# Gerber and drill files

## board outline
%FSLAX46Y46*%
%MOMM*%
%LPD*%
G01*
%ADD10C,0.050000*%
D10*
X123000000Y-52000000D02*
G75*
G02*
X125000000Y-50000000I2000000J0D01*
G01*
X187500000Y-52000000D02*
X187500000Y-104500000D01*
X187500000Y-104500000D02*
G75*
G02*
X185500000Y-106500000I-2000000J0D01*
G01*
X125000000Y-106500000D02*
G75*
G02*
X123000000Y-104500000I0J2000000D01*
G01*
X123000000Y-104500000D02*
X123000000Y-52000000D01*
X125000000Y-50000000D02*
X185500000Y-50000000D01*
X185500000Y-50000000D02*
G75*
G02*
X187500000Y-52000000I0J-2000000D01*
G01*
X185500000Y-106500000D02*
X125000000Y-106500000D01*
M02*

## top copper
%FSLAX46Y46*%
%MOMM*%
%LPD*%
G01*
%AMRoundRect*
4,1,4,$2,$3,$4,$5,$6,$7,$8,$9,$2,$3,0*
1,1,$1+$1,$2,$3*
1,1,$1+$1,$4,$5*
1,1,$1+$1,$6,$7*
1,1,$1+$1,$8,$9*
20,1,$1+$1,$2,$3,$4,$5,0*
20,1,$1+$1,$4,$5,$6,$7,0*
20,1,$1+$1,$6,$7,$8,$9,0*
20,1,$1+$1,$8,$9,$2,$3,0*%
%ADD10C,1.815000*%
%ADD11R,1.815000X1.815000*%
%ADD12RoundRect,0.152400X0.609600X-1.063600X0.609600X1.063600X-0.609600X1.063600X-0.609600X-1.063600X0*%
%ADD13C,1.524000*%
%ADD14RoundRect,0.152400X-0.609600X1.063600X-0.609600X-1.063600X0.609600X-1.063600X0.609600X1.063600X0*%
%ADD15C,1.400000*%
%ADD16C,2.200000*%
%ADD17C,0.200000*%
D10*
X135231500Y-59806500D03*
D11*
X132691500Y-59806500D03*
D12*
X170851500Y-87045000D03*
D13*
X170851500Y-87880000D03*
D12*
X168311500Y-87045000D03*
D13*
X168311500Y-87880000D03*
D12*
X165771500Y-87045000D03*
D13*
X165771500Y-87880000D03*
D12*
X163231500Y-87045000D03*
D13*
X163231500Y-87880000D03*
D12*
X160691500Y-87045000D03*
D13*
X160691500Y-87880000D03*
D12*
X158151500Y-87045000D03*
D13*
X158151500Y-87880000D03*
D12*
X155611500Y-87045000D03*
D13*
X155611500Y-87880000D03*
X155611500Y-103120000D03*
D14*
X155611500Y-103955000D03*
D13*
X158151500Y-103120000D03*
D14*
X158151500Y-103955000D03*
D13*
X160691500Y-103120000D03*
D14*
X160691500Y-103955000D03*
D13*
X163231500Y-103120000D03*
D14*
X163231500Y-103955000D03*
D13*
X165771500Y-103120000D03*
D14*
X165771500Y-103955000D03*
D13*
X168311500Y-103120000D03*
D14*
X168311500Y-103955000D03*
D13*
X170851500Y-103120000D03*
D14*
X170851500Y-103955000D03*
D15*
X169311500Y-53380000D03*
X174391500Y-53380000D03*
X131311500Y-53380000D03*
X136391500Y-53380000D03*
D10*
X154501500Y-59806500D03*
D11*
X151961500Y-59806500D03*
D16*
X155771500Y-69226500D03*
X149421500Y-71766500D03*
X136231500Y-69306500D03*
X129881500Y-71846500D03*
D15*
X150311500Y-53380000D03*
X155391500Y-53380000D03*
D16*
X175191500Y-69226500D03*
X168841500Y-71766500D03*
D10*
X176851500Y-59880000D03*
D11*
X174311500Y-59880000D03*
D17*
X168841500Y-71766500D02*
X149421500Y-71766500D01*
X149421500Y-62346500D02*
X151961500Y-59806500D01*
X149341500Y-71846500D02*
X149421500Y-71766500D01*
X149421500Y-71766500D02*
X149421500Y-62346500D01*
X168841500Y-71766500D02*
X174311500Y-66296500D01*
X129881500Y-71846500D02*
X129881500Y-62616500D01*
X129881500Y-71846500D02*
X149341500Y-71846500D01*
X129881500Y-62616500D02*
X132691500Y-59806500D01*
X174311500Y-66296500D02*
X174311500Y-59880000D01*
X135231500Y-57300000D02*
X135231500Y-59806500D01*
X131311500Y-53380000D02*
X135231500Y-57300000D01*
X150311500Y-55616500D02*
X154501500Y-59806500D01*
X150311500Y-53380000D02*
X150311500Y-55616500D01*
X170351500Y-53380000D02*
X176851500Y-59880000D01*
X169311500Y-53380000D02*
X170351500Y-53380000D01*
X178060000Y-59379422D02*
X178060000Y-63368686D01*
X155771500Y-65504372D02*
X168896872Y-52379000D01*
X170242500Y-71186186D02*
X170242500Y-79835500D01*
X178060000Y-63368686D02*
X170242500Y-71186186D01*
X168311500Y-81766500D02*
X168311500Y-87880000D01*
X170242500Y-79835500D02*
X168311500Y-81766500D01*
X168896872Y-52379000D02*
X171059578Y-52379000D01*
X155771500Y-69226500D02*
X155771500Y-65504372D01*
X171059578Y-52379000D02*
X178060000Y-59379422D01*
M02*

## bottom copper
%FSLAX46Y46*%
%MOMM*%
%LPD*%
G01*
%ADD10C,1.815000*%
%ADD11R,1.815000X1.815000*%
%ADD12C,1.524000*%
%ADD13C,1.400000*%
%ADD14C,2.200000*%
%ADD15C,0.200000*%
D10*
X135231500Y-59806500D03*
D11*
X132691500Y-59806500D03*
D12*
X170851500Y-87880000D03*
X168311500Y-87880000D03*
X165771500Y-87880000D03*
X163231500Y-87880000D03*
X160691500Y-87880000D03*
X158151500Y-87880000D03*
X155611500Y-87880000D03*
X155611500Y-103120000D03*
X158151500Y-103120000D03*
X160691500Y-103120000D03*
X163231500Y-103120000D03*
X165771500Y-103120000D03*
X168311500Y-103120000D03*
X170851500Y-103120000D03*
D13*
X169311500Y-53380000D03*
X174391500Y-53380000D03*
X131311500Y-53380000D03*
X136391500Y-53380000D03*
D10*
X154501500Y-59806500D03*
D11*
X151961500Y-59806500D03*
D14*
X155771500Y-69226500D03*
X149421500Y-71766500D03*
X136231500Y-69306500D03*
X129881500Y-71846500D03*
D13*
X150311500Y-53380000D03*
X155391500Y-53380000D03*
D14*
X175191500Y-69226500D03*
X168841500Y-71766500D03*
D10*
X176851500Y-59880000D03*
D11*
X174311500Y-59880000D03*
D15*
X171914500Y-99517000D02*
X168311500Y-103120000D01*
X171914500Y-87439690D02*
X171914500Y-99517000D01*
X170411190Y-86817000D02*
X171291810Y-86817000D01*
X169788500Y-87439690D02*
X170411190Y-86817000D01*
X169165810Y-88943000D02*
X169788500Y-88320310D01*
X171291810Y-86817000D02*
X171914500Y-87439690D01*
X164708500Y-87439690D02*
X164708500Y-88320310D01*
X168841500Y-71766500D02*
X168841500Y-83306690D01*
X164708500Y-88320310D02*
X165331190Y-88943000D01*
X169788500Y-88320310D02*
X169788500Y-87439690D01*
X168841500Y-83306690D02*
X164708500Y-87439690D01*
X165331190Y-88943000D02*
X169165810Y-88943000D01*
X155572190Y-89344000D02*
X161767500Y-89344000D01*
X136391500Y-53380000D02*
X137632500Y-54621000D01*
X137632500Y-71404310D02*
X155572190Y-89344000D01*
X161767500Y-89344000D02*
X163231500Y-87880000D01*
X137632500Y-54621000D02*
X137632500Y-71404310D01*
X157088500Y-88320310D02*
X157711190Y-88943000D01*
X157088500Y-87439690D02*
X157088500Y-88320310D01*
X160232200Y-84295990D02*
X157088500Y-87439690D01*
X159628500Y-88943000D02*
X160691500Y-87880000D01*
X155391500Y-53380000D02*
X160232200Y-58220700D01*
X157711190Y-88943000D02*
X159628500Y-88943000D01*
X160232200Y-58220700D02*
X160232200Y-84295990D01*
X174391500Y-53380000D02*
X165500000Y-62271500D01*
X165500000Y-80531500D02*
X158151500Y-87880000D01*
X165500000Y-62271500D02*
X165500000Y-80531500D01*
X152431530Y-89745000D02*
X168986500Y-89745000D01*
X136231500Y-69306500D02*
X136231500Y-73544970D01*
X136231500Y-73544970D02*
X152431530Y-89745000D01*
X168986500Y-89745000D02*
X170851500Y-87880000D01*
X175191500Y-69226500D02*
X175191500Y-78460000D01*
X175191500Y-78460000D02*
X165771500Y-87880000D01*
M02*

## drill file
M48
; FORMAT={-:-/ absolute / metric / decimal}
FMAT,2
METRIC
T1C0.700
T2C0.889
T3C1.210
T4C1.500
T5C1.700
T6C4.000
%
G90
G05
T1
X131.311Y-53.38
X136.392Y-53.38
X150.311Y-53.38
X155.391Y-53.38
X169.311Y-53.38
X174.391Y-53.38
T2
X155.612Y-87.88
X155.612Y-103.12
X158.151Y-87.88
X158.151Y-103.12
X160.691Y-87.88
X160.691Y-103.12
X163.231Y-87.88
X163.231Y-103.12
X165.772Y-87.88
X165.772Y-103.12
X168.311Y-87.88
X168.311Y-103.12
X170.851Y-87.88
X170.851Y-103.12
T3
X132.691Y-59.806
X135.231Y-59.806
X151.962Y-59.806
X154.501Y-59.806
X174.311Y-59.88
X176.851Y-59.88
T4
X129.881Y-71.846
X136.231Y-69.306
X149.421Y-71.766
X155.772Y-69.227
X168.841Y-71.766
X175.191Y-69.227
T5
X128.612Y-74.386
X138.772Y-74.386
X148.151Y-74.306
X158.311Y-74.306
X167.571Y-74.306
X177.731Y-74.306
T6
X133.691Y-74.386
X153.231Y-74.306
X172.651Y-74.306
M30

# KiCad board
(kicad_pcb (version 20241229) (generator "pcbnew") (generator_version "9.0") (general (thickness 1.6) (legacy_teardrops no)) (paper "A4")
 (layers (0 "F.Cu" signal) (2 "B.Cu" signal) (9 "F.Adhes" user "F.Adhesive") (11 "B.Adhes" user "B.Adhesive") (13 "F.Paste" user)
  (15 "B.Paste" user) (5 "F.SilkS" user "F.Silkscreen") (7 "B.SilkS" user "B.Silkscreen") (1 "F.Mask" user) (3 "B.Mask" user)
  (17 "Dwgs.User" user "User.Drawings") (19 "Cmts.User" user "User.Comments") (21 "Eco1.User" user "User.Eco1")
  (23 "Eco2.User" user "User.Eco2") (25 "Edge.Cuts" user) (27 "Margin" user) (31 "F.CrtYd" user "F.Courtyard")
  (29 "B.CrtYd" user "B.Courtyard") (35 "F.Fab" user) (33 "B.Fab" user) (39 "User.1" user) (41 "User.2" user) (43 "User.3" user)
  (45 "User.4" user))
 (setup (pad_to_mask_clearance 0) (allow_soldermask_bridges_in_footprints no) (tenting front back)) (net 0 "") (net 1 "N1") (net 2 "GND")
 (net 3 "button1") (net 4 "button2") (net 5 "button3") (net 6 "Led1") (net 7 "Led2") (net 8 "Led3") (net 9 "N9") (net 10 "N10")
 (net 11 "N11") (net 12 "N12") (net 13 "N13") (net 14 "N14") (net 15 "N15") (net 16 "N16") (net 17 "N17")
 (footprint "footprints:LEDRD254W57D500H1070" (layer "F.Cu") (at 133.9615 59.8065)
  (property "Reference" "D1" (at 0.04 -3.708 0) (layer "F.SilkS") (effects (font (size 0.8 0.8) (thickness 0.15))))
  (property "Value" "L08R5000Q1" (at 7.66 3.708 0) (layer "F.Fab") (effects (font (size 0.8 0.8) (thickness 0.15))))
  (pad "A" thru_hole circle (at 1.27 0) (size 1.815 1.815) (drill 1.21) (layers "*.Cu" "*.Mask") (remove_unused_layers no) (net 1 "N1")
   (solder_mask_margin 0.102))
  (pad "C" thru_hole rect (at -1.27 0) (size 1.815 1.815) (drill 1.21) (layers "*.Cu" "*.Mask") (remove_unused_layers no) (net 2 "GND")
   (solder_mask_margin 0.102)))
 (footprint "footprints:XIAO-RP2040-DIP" (layer "F.Cu") (at 163.2315 95.5 -90)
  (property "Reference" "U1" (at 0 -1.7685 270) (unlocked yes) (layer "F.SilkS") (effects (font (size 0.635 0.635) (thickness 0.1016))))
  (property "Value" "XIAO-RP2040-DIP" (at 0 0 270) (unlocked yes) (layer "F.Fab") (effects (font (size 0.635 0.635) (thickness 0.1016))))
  (pad "1" smd roundrect (at -8.455 -7.62 90) (size 2.432 1.524) (layers "F.Cu" "F.Mask") (roundrect_rratio 0.1) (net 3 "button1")
   (thermal_bridge_angle 45))
  (pad "1" thru_hole circle (at -7.62 -7.62 90) (size 1.524 1.524) (drill 0.889) (layers "*.Cu" "*.Mask") (remove_unused_layers no)
   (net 3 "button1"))
  (pad "2" smd roundrect (at -8.455 -5.08 90) (size 2.432 1.524) (layers "F.Cu" "F.Mask") (roundrect_rratio 0.1) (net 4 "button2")
   (thermal_bridge_angle 45))
  (pad "2" thru_hole circle (at -7.62 -5.08 90) (size 1.524 1.524) (drill 0.889) (layers "*.Cu" "*.Mask") (remove_unused_layers no)
   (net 4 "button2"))
  (pad "3" smd roundrect (at -8.455 -2.54 90) (size 2.432 1.524) (layers "F.Cu" "F.Mask") (roundrect_rratio 0.1) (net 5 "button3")
   (thermal_bridge_angle 45))
  (pad "3" thru_hole circle (at -7.62 -2.54 90) (size 1.524 1.524) (drill 0.889) (layers "*.Cu" "*.Mask") (remove_unused_layers no)
   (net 5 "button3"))
  (pad "4" smd roundrect (at -8.455 0 90) (size 2.432 1.524) (layers "F.Cu" "F.Mask") (roundrect_rratio 0.1) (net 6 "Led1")
   (thermal_bridge_angle 45))
  (pad "4" thru_hole circle (at -7.62 0 90) (size 1.524 1.524) (drill 0.889) (layers "*.Cu" "*.Mask") (remove_unused_layers no)
   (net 6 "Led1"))
  (pad "5" smd roundrect (at -8.455 2.54 90) (size 2.432 1.524) (layers "F.Cu" "F.Mask") (roundrect_rratio 0.1) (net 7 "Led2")
   (thermal_bridge_angle 45))
  (pad "5" thru_hole circle (at -7.62 2.54 90) (size 1.524 1.524) (drill 0.889) (layers "*.Cu" "*.Mask") (remove_unused_layers no)
   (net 7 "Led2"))
  (pad "6" smd roundrect (at -8.455 5.08 90) (size 2.432 1.524) (layers "F.Cu" "F.Mask") (roundrect_rratio 0.1) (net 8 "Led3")
   (thermal_bridge_angle 45))
  (pad "6" thru_hole circle (at -7.62 5.08 90) (size 1.524 1.524) (drill 0.889) (layers "*.Cu" "*.Mask") (remove_unused_layers no)
   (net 8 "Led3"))
  (pad "7" smd roundrect (at -8.455 7.62 90) (size 2.432 1.524) (layers "F.Cu" "F.Mask") (roundrect_rratio 0.1) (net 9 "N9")
   (thermal_bridge_angle 45))
  (pad "7" thru_hole circle (at -7.62 7.62 90) (size 1.524 1.524) (drill 0.889) (layers "*.Cu" "*.Mask") (remove_unused_layers no)
   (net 9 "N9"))
  (pad "8" thru_hole circle (at 7.62 7.62 270) (size 1.524 1.524) (drill 0.889) (layers "*.Cu" "*.Mask") (remove_unused_layers no)
   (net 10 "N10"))
  (pad "8" smd roundrect (at 8.455 7.62 270) (size 2.432 1.524) (layers "F.Cu" "F.Mask") (roundrect_rratio 0.1) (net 10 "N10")
   (thermal_bridge_angle 45))
  (pad "9" thru_hole circle (at 7.62 5.08 270) (size 1.524 1.524) (drill 0.889) (layers "*.Cu" "*.Mask") (remove_unused_layers no)
   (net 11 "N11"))
  (pad "9" smd roundrect (at 8.455 5.08 270) (size 2.432 1.524) (layers "F.Cu" "F.Mask") (roundrect_rratio 0.1) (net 11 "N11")
   (thermal_bridge_angle 45))
  (pad "10" thru_hole circle (at 7.62 2.54 270) (size 1.524 1.524) (drill 0.889) (layers "*.Cu" "*.Mask") (remove_unused_layers no)
   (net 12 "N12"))
  (pad "10" smd roundrect (at 8.455 2.54 270) (size 2.432 1.524) (layers "F.Cu" "F.Mask") (roundrect_rratio 0.1) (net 12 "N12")
   (thermal_bridge_angle 45))
  (pad "11" thru_hole circle (at 7.62 0 270) (size 1.524 1.524) (drill 0.889) (layers "*.Cu" "*.Mask") (remove_unused_layers no)
   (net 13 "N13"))
  (pad "11" smd roundrect (at 8.455 0 270) (size 2.432 1.524) (layers "F.Cu" "F.Mask") (roundrect_rratio 0.1) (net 13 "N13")
   (thermal_bridge_angle 45))
  (pad "12" thru_hole circle (at 7.62 -2.54 270) (size 1.524 1.524) (drill 0.889) (layers "*.Cu" "*.Mask") (remove_unused_layers no)
   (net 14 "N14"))
  (pad "12" smd roundrect (at 8.455 -2.54 270) (size 2.432 1.524) (layers "F.Cu" "F.Mask") (roundrect_rratio 0.1) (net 14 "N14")
   (thermal_bridge_angle 45))
  (pad "13" thru_hole circle (at 7.62 -5.08 270) (size 1.524 1.524) (drill 0.889) (layers "*.Cu" "*.Mask") (remove_unused_layers no)
   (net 2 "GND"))
  (pad "13" smd roundrect (at 8.455 -5.08 270) (size 2.432 1.524) (layers "F.Cu" "F.Mask") (roundrect_rratio 0.1) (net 2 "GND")
   (thermal_bridge_angle 45))
  (pad "14" thru_hole circle (at 7.62 -7.62 270) (size 1.524 1.524) (drill 0.889) (layers "*.Cu" "*.Mask") (remove_unused_layers no)
   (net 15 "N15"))
  (pad "14" smd roundrect (at 8.455 -7.62 270) (size 2.432 1.524) (layers "F.Cu" "F.Mask") (roundrect_rratio 0.1) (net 15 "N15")
   (thermal_bridge_angle 45)))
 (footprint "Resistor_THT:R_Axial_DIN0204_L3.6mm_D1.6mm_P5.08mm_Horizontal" (layer "F.Cu") (at 169.3115 53.38)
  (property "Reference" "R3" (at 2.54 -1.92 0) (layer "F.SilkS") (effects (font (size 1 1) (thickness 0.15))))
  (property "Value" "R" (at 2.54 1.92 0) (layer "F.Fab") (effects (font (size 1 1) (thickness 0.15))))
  (pad "1" thru_hole circle (at 0 0) (size 1.4 1.4) (drill 0.7) (layers "*.Cu" "*.Mask") (remove_unused_layers no) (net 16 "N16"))
  (pad "2" thru_hole circle (at 5.08 0) (size 1.4 1.4) (drill 0.7) (layers "*.Cu" "*.Mask") (remove_unused_layers no) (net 8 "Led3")))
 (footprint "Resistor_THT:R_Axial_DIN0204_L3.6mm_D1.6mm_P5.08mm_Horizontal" (layer "F.Cu") (at 131.3115 53.38)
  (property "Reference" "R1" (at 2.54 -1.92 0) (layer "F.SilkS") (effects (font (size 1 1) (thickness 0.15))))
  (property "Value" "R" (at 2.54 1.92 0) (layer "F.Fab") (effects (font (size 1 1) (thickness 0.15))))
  (pad "1" thru_hole circle (at 0 0) (size 1.4 1.4) (drill 0.7) (layers "*.Cu" "*.Mask") (remove_unused_layers no) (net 1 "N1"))
  (pad "2" thru_hole circle (at 5.08 0) (size 1.4 1.4) (drill 0.7) (layers "*.Cu" "*.Mask") (remove_unused_layers no) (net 6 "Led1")))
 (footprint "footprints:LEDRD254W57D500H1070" (layer "F.Cu") (at 153.2315 59.8065)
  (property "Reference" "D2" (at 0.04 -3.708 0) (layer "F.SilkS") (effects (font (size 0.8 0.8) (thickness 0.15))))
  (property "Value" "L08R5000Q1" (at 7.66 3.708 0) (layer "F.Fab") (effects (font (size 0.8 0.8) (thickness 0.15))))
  (pad "A" thru_hole circle (at 1.27 0) (size 1.815 1.815) (drill 1.21) (layers "*.Cu" "*.Mask") (remove_unused_layers no) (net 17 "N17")
   (solder_mask_margin 0.102))
  (pad "C" thru_hole rect (at -1.27 0) (size 1.815 1.815) (drill 1.21) (layers "*.Cu" "*.Mask") (remove_unused_layers no) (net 2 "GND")
   (solder_mask_margin 0.102)))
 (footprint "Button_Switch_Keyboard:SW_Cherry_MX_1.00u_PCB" (layer "F.Cu") (at 155.7715 69.2265)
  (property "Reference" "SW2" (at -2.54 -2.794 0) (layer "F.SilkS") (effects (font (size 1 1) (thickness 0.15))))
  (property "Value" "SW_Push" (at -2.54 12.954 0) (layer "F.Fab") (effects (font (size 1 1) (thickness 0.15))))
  (pad "" np_thru_hole circle (at -7.62 5.08) (size 1.7 1.7) (drill 1.7) (layers "*.Cu" "*.Mask"))
  (pad "" np_thru_hole circle (at -2.54 5.08) (size 4 4) (drill 4) (layers "*.Cu" "*.Mask"))
  (pad "" np_thru_hole circle (at 2.54 5.08) (size 1.7 1.7) (drill 1.7) (layers "*.Cu" "*.Mask"))
  (pad "1" thru_hole circle (at 0 0) (size 2.2 2.2) (drill 1.5) (layers "*.Cu" "*.Mask") (remove_unused_layers no) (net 4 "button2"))
  (pad "2" thru_hole circle (at -6.35 2.54) (size 2.2 2.2) (drill 1.5) (layers "*.Cu" "*.Mask") (remove_unused_layers no) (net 2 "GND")))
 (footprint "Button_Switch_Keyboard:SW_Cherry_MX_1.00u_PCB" (layer "F.Cu") (at 136.2315 69.3065)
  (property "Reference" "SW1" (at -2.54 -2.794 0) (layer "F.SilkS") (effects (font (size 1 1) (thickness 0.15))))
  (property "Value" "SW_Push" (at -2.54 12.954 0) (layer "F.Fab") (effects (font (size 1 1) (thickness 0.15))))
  (pad "" np_thru_hole circle (at -7.62 5.08) (size 1.7 1.7) (drill 1.7) (layers "*.Cu" "*.Mask"))
  (pad "" np_thru_hole circle (at -2.54 5.08) (size 4 4) (drill 4) (layers "*.Cu" "*.Mask"))
  (pad "" np_thru_hole circle (at 2.54 5.08) (size 1.7 1.7) (drill 1.7) (layers "*.Cu" "*.Mask"))
  (pad "1" thru_hole circle (at 0 0) (size 2.2 2.2) (drill 1.5) (layers "*.Cu" "*.Mask") (remove_unused_layers no) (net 3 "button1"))
  (pad "2" thru_hole circle (at -6.35 2.54) (size 2.2 2.2) (drill 1.5) (layers "*.Cu" "*.Mask") (remove_unused_layers no) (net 2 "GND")))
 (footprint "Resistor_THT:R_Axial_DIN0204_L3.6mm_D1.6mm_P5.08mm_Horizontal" (layer "F.Cu") (at 150.3115 53.38)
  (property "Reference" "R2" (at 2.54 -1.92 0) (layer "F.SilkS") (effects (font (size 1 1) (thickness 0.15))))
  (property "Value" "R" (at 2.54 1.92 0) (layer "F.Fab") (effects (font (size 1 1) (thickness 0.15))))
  (pad "1" thru_hole circle (at 0 0) (size 1.4 1.4) (drill 0.7) (layers "*.Cu" "*.Mask") (remove_unused_layers no) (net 17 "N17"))
  (pad "2" thru_hole circle (at 5.08 0) (size 1.4 1.4) (drill 0.7) (layers "*.Cu" "*.Mask") (remove_unused_layers no) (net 7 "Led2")))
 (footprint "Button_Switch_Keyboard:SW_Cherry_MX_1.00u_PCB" (layer "F.Cu") (at 175.1915 69.2265)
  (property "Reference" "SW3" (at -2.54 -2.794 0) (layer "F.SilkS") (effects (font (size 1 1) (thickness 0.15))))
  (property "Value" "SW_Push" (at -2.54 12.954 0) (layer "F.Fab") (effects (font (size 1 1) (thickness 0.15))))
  (pad "" np_thru_hole circle (at -7.62 5.08) (size 1.7 1.7) (drill 1.7) (layers "*.Cu" "*.Mask"))
  (pad "" np_thru_hole circle (at -2.54 5.08) (size 4 4) (drill 4) (layers "*.Cu" "*.Mask"))
  (pad "" np_thru_hole circle (at 2.54 5.08) (size 1.7 1.7) (drill 1.7) (layers "*.Cu" "*.Mask"))
  (pad "1" thru_hole circle (at 0 0) (size 2.2 2.2) (drill 1.5) (layers "*.Cu" "*.Mask") (remove_unused_layers no) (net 5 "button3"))
  (pad "2" thru_hole circle (at -6.35 2.54) (size 2.2 2.2) (drill 1.5) (layers "*.Cu" "*.Mask") (remove_unused_layers no) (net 2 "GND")))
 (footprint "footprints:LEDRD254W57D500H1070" (layer "F.Cu") (at 175.5815 59.88)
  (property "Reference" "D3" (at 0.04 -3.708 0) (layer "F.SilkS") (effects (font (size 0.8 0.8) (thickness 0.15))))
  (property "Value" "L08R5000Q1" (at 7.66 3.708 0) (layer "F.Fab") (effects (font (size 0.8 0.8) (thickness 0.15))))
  (pad "A" thru_hole circle (at 1.27 0) (size 1.815 1.815) (drill 1.21) (layers "*.Cu" "*.Mask") (remove_unused_layers no) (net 16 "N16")
   (solder_mask_margin 0.102))
  (pad "C" thru_hole rect (at -1.27 0) (size 1.815 1.815) (drill 1.21) (layers "*.Cu" "*.Mask") (remove_unused_layers no) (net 2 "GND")
   (solder_mask_margin 0.102)))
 (gr_arc (start 123 52) (mid 123.585786 50.585786) (end 125 50) (stroke (width 0.05) (type default)) (layer "Edge.Cuts"))
 (gr_line (start 187.5 52) (end 187.5 104.5) (stroke (width 0.05) (type default)) (layer "Edge.Cuts"))
 (gr_arc (start 187.5 104.5) (mid 186.914214 105.914214) (end 185.5 106.5) (stroke (width 0.05) (type default)) (layer "Edge.Cuts"))
 (gr_arc (start 125 106.5) (mid 123.585786 105.914214) (end 123 104.5) (stroke (width 0.05) (type default)) (layer "Edge.Cuts"))
 (gr_line (start 123 104.5) (end 123 52) (stroke (width 0.05) (type default)) (layer "Edge.Cuts"))
 (gr_line (start 125 50) (end 185.5 50) (stroke (width 0.05) (type default)) (layer "Edge.Cuts"))
 (gr_arc (start 185.5 50) (mid 186.914214 50.585786) (end 187.5 52) (stroke (width 0.05) (type default)) (layer "Edge.Cuts"))
 (gr_line (start 185.5 106.5) (end 125 106.5) (stroke (width 0.05) (type default)) (layer "Edge.Cuts"))
 (segment (start 168.8415 71.7665) (end 149.4215 71.7665) (width 0.2) (layer "F.Cu") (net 2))
 (segment (start 149.4215 62.3465) (end 151.9615 59.8065) (width 0.2) (layer "F.Cu") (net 2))
 (segment (start 149.3415 71.8465) (end 149.4215 71.7665) (width 0.2) (layer "F.Cu") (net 2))
 (segment (start 149.4215 71.7665) (end 149.4215 62.3465) (width 0.2) (layer "F.Cu") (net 2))
 (segment (start 168.8415 71.7665) (end 174.3115 66.2965) (width 0.2) (layer "F.Cu") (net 2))
 (segment (start 129.8815 71.8465) (end 129.8815 62.6165) (width 0.2) (layer "F.Cu") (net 2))
 (segment (start 129.8815 71.8465) (end 149.3415 71.8465) (width 0.2) (layer "F.Cu") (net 2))
 (segment (start 129.8815 62.6165) (end 132.6915 59.8065) (width 0.2) (layer "F.Cu") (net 2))
 (segment (start 174.3115 66.2965) (end 174.3115 59.88) (width 0.2) (layer "F.Cu") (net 2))
 (segment (start 171.9145 99.517) (end 168.3115 103.12) (width 0.2) (layer "B.Cu") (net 2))
 (segment (start 171.9145 87.43969) (end 171.9145 99.517) (width 0.2) (layer "B.Cu") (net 2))
 (segment (start 170.41119 86.817) (end 171.29181 86.817) (width 0.2) (layer "B.Cu") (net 2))
 (segment (start 169.7885 87.43969) (end 170.41119 86.817) (width 0.2) (layer "B.Cu") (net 2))
 (segment (start 169.16581 88.943) (end 169.7885 88.32031) (width 0.2) (layer "B.Cu") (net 2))
 (segment (start 171.29181 86.817) (end 171.9145 87.43969) (width 0.2) (layer "B.Cu") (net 2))
 (segment (start 164.7085 87.43969) (end 164.7085 88.32031) (width 0.2) (layer "B.Cu") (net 2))
 (segment (start 168.8415 71.7665) (end 168.8415 83.30669) (width 0.2) (layer "B.Cu") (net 2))
 (segment (start 164.7085 88.32031) (end 165.33119 88.943) (width 0.2) (layer "B.Cu") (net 2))
 (segment (start 169.7885 88.32031) (end 169.7885 87.43969) (width 0.2) (layer "B.Cu") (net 2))
 (segment (start 168.8415 83.30669) (end 164.7085 87.43969) (width 0.2) (layer "B.Cu") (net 2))
 (segment (start 165.33119 88.943) (end 169.16581 88.943) (width 0.2) (layer "B.Cu") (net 2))
 (segment (start 135.2315 57.3) (end 135.2315 59.8065) (width 0.2) (layer "F.Cu") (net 1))
 (segment (start 131.3115 53.38) (end 135.2315 57.3) (width 0.2) (layer "F.Cu") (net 1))
 (segment (start 150.3115 55.6165) (end 154.5015 59.8065) (width 0.2) (layer "F.Cu") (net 17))
 (segment (start 150.3115 53.38) (end 150.3115 55.6165) (width 0.2) (layer "F.Cu") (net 17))
 (segment (start 170.3515 53.38) (end 176.8515 59.88) (width 0.2) (layer "F.Cu") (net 16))
 (segment (start 169.3115 53.38) (end 170.3515 53.38) (width 0.2) (layer "F.Cu") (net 16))
 (segment (start 155.57219 89.344) (end 161.7675 89.344) (width 0.2) (layer "B.Cu") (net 6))
 (segment (start 136.3915 53.38) (end 137.6325 54.621) (width 0.2) (layer "B.Cu") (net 6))
 (segment (start 137.6325 71.40431) (end 155.57219 89.344) (width 0.2) (layer "B.Cu") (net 6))
 (segment (start 161.7675 89.344) (end 163.2315 87.88) (width 0.2) (layer "B.Cu") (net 6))
 (segment (start 137.6325 54.621) (end 137.6325 71.40431) (width 0.2) (layer "B.Cu") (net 6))
 (segment (start 157.0885 88.32031) (end 157.71119 88.943) (width 0.2) (layer "B.Cu") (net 7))
 (segment (start 157.0885 87.43969) (end 157.0885 88.32031) (width 0.2) (layer "B.Cu") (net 7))
 (segment (start 160.2322 84.29599) (end 157.0885 87.43969) (width 0.2) (layer "B.Cu") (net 7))
 (segment (start 159.6285 88.943) (end 160.6915 87.88) (width 0.2) (layer "B.Cu") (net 7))
 (segment (start 155.3915 53.38) (end 160.2322 58.2207) (width 0.2) (layer "B.Cu") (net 7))
 (segment (start 157.71119 88.943) (end 159.6285 88.943) (width 0.2) (layer "B.Cu") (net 7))
 (segment (start 160.2322 58.2207) (end 160.2322 84.29599) (width 0.2) (layer "B.Cu") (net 7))
 (segment (start 174.3915 53.38) (end 165.5 62.2715) (width 0.2) (layer "B.Cu") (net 8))
 (segment (start 165.5 80.5315) (end 158.1515 87.88) (width 0.2) (layer "B.Cu") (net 8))
 (segment (start 165.5 62.2715) (end 165.5 80.5315) (width 0.2) (layer "B.Cu") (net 8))
 (segment (start 152.43153 89.745) (end 168.9865 89.745) (width 0.2) (layer "B.Cu") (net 3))
 (segment (start 136.2315 69.3065) (end 136.2315 73.54497) (width 0.2) (layer "B.Cu") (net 3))
 (segment (start 136.2315 73.54497) (end 152.43153 89.745) (width 0.2) (layer "B.Cu") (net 3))
 (segment (start 168.9865 89.745) (end 170.8515 87.88) (width 0.2) (layer "B.Cu") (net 3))
 (segment (start 178.06 59.379422) (end 178.06 63.368686) (width 0.2) (layer "F.Cu") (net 4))
 (segment (start 155.7715 65.504372) (end 168.896872 52.379) (width 0.2) (layer "F.Cu") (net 4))
 (segment (start 170.2425 71.186186) (end 170.2425 79.8355) (width 0.2) (layer "F.Cu") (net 4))
 (segment (start 178.06 63.368686) (end 170.2425 71.186186) (width 0.2) (layer "F.Cu") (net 4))
 (segment (start 168.3115 81.7665) (end 168.3115 87.88) (width 0.2) (layer "F.Cu") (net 4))
 (segment (start 170.2425 79.8355) (end 168.3115 81.7665) (width 0.2) (layer "F.Cu") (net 4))
 (segment (start 168.896872 52.379) (end 171.059578 52.379) (width 0.2) (layer "F.Cu") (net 4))
 (segment (start 155.7715 69.2265) (end 155.7715 65.504372) (width 0.2) (layer "F.Cu") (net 4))
 (segment (start 171.059578 52.379) (end 178.06 59.379422) (width 0.2) (layer "F.Cu") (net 4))
 (segment (start 175.1915 69.2265) (end 175.1915 78.46) (width 0.2) (layer "B.Cu") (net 5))
 (segment (start 175.1915 78.46) (end 165.7715 87.88) (width 0.2) (layer "B.Cu") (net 5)))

